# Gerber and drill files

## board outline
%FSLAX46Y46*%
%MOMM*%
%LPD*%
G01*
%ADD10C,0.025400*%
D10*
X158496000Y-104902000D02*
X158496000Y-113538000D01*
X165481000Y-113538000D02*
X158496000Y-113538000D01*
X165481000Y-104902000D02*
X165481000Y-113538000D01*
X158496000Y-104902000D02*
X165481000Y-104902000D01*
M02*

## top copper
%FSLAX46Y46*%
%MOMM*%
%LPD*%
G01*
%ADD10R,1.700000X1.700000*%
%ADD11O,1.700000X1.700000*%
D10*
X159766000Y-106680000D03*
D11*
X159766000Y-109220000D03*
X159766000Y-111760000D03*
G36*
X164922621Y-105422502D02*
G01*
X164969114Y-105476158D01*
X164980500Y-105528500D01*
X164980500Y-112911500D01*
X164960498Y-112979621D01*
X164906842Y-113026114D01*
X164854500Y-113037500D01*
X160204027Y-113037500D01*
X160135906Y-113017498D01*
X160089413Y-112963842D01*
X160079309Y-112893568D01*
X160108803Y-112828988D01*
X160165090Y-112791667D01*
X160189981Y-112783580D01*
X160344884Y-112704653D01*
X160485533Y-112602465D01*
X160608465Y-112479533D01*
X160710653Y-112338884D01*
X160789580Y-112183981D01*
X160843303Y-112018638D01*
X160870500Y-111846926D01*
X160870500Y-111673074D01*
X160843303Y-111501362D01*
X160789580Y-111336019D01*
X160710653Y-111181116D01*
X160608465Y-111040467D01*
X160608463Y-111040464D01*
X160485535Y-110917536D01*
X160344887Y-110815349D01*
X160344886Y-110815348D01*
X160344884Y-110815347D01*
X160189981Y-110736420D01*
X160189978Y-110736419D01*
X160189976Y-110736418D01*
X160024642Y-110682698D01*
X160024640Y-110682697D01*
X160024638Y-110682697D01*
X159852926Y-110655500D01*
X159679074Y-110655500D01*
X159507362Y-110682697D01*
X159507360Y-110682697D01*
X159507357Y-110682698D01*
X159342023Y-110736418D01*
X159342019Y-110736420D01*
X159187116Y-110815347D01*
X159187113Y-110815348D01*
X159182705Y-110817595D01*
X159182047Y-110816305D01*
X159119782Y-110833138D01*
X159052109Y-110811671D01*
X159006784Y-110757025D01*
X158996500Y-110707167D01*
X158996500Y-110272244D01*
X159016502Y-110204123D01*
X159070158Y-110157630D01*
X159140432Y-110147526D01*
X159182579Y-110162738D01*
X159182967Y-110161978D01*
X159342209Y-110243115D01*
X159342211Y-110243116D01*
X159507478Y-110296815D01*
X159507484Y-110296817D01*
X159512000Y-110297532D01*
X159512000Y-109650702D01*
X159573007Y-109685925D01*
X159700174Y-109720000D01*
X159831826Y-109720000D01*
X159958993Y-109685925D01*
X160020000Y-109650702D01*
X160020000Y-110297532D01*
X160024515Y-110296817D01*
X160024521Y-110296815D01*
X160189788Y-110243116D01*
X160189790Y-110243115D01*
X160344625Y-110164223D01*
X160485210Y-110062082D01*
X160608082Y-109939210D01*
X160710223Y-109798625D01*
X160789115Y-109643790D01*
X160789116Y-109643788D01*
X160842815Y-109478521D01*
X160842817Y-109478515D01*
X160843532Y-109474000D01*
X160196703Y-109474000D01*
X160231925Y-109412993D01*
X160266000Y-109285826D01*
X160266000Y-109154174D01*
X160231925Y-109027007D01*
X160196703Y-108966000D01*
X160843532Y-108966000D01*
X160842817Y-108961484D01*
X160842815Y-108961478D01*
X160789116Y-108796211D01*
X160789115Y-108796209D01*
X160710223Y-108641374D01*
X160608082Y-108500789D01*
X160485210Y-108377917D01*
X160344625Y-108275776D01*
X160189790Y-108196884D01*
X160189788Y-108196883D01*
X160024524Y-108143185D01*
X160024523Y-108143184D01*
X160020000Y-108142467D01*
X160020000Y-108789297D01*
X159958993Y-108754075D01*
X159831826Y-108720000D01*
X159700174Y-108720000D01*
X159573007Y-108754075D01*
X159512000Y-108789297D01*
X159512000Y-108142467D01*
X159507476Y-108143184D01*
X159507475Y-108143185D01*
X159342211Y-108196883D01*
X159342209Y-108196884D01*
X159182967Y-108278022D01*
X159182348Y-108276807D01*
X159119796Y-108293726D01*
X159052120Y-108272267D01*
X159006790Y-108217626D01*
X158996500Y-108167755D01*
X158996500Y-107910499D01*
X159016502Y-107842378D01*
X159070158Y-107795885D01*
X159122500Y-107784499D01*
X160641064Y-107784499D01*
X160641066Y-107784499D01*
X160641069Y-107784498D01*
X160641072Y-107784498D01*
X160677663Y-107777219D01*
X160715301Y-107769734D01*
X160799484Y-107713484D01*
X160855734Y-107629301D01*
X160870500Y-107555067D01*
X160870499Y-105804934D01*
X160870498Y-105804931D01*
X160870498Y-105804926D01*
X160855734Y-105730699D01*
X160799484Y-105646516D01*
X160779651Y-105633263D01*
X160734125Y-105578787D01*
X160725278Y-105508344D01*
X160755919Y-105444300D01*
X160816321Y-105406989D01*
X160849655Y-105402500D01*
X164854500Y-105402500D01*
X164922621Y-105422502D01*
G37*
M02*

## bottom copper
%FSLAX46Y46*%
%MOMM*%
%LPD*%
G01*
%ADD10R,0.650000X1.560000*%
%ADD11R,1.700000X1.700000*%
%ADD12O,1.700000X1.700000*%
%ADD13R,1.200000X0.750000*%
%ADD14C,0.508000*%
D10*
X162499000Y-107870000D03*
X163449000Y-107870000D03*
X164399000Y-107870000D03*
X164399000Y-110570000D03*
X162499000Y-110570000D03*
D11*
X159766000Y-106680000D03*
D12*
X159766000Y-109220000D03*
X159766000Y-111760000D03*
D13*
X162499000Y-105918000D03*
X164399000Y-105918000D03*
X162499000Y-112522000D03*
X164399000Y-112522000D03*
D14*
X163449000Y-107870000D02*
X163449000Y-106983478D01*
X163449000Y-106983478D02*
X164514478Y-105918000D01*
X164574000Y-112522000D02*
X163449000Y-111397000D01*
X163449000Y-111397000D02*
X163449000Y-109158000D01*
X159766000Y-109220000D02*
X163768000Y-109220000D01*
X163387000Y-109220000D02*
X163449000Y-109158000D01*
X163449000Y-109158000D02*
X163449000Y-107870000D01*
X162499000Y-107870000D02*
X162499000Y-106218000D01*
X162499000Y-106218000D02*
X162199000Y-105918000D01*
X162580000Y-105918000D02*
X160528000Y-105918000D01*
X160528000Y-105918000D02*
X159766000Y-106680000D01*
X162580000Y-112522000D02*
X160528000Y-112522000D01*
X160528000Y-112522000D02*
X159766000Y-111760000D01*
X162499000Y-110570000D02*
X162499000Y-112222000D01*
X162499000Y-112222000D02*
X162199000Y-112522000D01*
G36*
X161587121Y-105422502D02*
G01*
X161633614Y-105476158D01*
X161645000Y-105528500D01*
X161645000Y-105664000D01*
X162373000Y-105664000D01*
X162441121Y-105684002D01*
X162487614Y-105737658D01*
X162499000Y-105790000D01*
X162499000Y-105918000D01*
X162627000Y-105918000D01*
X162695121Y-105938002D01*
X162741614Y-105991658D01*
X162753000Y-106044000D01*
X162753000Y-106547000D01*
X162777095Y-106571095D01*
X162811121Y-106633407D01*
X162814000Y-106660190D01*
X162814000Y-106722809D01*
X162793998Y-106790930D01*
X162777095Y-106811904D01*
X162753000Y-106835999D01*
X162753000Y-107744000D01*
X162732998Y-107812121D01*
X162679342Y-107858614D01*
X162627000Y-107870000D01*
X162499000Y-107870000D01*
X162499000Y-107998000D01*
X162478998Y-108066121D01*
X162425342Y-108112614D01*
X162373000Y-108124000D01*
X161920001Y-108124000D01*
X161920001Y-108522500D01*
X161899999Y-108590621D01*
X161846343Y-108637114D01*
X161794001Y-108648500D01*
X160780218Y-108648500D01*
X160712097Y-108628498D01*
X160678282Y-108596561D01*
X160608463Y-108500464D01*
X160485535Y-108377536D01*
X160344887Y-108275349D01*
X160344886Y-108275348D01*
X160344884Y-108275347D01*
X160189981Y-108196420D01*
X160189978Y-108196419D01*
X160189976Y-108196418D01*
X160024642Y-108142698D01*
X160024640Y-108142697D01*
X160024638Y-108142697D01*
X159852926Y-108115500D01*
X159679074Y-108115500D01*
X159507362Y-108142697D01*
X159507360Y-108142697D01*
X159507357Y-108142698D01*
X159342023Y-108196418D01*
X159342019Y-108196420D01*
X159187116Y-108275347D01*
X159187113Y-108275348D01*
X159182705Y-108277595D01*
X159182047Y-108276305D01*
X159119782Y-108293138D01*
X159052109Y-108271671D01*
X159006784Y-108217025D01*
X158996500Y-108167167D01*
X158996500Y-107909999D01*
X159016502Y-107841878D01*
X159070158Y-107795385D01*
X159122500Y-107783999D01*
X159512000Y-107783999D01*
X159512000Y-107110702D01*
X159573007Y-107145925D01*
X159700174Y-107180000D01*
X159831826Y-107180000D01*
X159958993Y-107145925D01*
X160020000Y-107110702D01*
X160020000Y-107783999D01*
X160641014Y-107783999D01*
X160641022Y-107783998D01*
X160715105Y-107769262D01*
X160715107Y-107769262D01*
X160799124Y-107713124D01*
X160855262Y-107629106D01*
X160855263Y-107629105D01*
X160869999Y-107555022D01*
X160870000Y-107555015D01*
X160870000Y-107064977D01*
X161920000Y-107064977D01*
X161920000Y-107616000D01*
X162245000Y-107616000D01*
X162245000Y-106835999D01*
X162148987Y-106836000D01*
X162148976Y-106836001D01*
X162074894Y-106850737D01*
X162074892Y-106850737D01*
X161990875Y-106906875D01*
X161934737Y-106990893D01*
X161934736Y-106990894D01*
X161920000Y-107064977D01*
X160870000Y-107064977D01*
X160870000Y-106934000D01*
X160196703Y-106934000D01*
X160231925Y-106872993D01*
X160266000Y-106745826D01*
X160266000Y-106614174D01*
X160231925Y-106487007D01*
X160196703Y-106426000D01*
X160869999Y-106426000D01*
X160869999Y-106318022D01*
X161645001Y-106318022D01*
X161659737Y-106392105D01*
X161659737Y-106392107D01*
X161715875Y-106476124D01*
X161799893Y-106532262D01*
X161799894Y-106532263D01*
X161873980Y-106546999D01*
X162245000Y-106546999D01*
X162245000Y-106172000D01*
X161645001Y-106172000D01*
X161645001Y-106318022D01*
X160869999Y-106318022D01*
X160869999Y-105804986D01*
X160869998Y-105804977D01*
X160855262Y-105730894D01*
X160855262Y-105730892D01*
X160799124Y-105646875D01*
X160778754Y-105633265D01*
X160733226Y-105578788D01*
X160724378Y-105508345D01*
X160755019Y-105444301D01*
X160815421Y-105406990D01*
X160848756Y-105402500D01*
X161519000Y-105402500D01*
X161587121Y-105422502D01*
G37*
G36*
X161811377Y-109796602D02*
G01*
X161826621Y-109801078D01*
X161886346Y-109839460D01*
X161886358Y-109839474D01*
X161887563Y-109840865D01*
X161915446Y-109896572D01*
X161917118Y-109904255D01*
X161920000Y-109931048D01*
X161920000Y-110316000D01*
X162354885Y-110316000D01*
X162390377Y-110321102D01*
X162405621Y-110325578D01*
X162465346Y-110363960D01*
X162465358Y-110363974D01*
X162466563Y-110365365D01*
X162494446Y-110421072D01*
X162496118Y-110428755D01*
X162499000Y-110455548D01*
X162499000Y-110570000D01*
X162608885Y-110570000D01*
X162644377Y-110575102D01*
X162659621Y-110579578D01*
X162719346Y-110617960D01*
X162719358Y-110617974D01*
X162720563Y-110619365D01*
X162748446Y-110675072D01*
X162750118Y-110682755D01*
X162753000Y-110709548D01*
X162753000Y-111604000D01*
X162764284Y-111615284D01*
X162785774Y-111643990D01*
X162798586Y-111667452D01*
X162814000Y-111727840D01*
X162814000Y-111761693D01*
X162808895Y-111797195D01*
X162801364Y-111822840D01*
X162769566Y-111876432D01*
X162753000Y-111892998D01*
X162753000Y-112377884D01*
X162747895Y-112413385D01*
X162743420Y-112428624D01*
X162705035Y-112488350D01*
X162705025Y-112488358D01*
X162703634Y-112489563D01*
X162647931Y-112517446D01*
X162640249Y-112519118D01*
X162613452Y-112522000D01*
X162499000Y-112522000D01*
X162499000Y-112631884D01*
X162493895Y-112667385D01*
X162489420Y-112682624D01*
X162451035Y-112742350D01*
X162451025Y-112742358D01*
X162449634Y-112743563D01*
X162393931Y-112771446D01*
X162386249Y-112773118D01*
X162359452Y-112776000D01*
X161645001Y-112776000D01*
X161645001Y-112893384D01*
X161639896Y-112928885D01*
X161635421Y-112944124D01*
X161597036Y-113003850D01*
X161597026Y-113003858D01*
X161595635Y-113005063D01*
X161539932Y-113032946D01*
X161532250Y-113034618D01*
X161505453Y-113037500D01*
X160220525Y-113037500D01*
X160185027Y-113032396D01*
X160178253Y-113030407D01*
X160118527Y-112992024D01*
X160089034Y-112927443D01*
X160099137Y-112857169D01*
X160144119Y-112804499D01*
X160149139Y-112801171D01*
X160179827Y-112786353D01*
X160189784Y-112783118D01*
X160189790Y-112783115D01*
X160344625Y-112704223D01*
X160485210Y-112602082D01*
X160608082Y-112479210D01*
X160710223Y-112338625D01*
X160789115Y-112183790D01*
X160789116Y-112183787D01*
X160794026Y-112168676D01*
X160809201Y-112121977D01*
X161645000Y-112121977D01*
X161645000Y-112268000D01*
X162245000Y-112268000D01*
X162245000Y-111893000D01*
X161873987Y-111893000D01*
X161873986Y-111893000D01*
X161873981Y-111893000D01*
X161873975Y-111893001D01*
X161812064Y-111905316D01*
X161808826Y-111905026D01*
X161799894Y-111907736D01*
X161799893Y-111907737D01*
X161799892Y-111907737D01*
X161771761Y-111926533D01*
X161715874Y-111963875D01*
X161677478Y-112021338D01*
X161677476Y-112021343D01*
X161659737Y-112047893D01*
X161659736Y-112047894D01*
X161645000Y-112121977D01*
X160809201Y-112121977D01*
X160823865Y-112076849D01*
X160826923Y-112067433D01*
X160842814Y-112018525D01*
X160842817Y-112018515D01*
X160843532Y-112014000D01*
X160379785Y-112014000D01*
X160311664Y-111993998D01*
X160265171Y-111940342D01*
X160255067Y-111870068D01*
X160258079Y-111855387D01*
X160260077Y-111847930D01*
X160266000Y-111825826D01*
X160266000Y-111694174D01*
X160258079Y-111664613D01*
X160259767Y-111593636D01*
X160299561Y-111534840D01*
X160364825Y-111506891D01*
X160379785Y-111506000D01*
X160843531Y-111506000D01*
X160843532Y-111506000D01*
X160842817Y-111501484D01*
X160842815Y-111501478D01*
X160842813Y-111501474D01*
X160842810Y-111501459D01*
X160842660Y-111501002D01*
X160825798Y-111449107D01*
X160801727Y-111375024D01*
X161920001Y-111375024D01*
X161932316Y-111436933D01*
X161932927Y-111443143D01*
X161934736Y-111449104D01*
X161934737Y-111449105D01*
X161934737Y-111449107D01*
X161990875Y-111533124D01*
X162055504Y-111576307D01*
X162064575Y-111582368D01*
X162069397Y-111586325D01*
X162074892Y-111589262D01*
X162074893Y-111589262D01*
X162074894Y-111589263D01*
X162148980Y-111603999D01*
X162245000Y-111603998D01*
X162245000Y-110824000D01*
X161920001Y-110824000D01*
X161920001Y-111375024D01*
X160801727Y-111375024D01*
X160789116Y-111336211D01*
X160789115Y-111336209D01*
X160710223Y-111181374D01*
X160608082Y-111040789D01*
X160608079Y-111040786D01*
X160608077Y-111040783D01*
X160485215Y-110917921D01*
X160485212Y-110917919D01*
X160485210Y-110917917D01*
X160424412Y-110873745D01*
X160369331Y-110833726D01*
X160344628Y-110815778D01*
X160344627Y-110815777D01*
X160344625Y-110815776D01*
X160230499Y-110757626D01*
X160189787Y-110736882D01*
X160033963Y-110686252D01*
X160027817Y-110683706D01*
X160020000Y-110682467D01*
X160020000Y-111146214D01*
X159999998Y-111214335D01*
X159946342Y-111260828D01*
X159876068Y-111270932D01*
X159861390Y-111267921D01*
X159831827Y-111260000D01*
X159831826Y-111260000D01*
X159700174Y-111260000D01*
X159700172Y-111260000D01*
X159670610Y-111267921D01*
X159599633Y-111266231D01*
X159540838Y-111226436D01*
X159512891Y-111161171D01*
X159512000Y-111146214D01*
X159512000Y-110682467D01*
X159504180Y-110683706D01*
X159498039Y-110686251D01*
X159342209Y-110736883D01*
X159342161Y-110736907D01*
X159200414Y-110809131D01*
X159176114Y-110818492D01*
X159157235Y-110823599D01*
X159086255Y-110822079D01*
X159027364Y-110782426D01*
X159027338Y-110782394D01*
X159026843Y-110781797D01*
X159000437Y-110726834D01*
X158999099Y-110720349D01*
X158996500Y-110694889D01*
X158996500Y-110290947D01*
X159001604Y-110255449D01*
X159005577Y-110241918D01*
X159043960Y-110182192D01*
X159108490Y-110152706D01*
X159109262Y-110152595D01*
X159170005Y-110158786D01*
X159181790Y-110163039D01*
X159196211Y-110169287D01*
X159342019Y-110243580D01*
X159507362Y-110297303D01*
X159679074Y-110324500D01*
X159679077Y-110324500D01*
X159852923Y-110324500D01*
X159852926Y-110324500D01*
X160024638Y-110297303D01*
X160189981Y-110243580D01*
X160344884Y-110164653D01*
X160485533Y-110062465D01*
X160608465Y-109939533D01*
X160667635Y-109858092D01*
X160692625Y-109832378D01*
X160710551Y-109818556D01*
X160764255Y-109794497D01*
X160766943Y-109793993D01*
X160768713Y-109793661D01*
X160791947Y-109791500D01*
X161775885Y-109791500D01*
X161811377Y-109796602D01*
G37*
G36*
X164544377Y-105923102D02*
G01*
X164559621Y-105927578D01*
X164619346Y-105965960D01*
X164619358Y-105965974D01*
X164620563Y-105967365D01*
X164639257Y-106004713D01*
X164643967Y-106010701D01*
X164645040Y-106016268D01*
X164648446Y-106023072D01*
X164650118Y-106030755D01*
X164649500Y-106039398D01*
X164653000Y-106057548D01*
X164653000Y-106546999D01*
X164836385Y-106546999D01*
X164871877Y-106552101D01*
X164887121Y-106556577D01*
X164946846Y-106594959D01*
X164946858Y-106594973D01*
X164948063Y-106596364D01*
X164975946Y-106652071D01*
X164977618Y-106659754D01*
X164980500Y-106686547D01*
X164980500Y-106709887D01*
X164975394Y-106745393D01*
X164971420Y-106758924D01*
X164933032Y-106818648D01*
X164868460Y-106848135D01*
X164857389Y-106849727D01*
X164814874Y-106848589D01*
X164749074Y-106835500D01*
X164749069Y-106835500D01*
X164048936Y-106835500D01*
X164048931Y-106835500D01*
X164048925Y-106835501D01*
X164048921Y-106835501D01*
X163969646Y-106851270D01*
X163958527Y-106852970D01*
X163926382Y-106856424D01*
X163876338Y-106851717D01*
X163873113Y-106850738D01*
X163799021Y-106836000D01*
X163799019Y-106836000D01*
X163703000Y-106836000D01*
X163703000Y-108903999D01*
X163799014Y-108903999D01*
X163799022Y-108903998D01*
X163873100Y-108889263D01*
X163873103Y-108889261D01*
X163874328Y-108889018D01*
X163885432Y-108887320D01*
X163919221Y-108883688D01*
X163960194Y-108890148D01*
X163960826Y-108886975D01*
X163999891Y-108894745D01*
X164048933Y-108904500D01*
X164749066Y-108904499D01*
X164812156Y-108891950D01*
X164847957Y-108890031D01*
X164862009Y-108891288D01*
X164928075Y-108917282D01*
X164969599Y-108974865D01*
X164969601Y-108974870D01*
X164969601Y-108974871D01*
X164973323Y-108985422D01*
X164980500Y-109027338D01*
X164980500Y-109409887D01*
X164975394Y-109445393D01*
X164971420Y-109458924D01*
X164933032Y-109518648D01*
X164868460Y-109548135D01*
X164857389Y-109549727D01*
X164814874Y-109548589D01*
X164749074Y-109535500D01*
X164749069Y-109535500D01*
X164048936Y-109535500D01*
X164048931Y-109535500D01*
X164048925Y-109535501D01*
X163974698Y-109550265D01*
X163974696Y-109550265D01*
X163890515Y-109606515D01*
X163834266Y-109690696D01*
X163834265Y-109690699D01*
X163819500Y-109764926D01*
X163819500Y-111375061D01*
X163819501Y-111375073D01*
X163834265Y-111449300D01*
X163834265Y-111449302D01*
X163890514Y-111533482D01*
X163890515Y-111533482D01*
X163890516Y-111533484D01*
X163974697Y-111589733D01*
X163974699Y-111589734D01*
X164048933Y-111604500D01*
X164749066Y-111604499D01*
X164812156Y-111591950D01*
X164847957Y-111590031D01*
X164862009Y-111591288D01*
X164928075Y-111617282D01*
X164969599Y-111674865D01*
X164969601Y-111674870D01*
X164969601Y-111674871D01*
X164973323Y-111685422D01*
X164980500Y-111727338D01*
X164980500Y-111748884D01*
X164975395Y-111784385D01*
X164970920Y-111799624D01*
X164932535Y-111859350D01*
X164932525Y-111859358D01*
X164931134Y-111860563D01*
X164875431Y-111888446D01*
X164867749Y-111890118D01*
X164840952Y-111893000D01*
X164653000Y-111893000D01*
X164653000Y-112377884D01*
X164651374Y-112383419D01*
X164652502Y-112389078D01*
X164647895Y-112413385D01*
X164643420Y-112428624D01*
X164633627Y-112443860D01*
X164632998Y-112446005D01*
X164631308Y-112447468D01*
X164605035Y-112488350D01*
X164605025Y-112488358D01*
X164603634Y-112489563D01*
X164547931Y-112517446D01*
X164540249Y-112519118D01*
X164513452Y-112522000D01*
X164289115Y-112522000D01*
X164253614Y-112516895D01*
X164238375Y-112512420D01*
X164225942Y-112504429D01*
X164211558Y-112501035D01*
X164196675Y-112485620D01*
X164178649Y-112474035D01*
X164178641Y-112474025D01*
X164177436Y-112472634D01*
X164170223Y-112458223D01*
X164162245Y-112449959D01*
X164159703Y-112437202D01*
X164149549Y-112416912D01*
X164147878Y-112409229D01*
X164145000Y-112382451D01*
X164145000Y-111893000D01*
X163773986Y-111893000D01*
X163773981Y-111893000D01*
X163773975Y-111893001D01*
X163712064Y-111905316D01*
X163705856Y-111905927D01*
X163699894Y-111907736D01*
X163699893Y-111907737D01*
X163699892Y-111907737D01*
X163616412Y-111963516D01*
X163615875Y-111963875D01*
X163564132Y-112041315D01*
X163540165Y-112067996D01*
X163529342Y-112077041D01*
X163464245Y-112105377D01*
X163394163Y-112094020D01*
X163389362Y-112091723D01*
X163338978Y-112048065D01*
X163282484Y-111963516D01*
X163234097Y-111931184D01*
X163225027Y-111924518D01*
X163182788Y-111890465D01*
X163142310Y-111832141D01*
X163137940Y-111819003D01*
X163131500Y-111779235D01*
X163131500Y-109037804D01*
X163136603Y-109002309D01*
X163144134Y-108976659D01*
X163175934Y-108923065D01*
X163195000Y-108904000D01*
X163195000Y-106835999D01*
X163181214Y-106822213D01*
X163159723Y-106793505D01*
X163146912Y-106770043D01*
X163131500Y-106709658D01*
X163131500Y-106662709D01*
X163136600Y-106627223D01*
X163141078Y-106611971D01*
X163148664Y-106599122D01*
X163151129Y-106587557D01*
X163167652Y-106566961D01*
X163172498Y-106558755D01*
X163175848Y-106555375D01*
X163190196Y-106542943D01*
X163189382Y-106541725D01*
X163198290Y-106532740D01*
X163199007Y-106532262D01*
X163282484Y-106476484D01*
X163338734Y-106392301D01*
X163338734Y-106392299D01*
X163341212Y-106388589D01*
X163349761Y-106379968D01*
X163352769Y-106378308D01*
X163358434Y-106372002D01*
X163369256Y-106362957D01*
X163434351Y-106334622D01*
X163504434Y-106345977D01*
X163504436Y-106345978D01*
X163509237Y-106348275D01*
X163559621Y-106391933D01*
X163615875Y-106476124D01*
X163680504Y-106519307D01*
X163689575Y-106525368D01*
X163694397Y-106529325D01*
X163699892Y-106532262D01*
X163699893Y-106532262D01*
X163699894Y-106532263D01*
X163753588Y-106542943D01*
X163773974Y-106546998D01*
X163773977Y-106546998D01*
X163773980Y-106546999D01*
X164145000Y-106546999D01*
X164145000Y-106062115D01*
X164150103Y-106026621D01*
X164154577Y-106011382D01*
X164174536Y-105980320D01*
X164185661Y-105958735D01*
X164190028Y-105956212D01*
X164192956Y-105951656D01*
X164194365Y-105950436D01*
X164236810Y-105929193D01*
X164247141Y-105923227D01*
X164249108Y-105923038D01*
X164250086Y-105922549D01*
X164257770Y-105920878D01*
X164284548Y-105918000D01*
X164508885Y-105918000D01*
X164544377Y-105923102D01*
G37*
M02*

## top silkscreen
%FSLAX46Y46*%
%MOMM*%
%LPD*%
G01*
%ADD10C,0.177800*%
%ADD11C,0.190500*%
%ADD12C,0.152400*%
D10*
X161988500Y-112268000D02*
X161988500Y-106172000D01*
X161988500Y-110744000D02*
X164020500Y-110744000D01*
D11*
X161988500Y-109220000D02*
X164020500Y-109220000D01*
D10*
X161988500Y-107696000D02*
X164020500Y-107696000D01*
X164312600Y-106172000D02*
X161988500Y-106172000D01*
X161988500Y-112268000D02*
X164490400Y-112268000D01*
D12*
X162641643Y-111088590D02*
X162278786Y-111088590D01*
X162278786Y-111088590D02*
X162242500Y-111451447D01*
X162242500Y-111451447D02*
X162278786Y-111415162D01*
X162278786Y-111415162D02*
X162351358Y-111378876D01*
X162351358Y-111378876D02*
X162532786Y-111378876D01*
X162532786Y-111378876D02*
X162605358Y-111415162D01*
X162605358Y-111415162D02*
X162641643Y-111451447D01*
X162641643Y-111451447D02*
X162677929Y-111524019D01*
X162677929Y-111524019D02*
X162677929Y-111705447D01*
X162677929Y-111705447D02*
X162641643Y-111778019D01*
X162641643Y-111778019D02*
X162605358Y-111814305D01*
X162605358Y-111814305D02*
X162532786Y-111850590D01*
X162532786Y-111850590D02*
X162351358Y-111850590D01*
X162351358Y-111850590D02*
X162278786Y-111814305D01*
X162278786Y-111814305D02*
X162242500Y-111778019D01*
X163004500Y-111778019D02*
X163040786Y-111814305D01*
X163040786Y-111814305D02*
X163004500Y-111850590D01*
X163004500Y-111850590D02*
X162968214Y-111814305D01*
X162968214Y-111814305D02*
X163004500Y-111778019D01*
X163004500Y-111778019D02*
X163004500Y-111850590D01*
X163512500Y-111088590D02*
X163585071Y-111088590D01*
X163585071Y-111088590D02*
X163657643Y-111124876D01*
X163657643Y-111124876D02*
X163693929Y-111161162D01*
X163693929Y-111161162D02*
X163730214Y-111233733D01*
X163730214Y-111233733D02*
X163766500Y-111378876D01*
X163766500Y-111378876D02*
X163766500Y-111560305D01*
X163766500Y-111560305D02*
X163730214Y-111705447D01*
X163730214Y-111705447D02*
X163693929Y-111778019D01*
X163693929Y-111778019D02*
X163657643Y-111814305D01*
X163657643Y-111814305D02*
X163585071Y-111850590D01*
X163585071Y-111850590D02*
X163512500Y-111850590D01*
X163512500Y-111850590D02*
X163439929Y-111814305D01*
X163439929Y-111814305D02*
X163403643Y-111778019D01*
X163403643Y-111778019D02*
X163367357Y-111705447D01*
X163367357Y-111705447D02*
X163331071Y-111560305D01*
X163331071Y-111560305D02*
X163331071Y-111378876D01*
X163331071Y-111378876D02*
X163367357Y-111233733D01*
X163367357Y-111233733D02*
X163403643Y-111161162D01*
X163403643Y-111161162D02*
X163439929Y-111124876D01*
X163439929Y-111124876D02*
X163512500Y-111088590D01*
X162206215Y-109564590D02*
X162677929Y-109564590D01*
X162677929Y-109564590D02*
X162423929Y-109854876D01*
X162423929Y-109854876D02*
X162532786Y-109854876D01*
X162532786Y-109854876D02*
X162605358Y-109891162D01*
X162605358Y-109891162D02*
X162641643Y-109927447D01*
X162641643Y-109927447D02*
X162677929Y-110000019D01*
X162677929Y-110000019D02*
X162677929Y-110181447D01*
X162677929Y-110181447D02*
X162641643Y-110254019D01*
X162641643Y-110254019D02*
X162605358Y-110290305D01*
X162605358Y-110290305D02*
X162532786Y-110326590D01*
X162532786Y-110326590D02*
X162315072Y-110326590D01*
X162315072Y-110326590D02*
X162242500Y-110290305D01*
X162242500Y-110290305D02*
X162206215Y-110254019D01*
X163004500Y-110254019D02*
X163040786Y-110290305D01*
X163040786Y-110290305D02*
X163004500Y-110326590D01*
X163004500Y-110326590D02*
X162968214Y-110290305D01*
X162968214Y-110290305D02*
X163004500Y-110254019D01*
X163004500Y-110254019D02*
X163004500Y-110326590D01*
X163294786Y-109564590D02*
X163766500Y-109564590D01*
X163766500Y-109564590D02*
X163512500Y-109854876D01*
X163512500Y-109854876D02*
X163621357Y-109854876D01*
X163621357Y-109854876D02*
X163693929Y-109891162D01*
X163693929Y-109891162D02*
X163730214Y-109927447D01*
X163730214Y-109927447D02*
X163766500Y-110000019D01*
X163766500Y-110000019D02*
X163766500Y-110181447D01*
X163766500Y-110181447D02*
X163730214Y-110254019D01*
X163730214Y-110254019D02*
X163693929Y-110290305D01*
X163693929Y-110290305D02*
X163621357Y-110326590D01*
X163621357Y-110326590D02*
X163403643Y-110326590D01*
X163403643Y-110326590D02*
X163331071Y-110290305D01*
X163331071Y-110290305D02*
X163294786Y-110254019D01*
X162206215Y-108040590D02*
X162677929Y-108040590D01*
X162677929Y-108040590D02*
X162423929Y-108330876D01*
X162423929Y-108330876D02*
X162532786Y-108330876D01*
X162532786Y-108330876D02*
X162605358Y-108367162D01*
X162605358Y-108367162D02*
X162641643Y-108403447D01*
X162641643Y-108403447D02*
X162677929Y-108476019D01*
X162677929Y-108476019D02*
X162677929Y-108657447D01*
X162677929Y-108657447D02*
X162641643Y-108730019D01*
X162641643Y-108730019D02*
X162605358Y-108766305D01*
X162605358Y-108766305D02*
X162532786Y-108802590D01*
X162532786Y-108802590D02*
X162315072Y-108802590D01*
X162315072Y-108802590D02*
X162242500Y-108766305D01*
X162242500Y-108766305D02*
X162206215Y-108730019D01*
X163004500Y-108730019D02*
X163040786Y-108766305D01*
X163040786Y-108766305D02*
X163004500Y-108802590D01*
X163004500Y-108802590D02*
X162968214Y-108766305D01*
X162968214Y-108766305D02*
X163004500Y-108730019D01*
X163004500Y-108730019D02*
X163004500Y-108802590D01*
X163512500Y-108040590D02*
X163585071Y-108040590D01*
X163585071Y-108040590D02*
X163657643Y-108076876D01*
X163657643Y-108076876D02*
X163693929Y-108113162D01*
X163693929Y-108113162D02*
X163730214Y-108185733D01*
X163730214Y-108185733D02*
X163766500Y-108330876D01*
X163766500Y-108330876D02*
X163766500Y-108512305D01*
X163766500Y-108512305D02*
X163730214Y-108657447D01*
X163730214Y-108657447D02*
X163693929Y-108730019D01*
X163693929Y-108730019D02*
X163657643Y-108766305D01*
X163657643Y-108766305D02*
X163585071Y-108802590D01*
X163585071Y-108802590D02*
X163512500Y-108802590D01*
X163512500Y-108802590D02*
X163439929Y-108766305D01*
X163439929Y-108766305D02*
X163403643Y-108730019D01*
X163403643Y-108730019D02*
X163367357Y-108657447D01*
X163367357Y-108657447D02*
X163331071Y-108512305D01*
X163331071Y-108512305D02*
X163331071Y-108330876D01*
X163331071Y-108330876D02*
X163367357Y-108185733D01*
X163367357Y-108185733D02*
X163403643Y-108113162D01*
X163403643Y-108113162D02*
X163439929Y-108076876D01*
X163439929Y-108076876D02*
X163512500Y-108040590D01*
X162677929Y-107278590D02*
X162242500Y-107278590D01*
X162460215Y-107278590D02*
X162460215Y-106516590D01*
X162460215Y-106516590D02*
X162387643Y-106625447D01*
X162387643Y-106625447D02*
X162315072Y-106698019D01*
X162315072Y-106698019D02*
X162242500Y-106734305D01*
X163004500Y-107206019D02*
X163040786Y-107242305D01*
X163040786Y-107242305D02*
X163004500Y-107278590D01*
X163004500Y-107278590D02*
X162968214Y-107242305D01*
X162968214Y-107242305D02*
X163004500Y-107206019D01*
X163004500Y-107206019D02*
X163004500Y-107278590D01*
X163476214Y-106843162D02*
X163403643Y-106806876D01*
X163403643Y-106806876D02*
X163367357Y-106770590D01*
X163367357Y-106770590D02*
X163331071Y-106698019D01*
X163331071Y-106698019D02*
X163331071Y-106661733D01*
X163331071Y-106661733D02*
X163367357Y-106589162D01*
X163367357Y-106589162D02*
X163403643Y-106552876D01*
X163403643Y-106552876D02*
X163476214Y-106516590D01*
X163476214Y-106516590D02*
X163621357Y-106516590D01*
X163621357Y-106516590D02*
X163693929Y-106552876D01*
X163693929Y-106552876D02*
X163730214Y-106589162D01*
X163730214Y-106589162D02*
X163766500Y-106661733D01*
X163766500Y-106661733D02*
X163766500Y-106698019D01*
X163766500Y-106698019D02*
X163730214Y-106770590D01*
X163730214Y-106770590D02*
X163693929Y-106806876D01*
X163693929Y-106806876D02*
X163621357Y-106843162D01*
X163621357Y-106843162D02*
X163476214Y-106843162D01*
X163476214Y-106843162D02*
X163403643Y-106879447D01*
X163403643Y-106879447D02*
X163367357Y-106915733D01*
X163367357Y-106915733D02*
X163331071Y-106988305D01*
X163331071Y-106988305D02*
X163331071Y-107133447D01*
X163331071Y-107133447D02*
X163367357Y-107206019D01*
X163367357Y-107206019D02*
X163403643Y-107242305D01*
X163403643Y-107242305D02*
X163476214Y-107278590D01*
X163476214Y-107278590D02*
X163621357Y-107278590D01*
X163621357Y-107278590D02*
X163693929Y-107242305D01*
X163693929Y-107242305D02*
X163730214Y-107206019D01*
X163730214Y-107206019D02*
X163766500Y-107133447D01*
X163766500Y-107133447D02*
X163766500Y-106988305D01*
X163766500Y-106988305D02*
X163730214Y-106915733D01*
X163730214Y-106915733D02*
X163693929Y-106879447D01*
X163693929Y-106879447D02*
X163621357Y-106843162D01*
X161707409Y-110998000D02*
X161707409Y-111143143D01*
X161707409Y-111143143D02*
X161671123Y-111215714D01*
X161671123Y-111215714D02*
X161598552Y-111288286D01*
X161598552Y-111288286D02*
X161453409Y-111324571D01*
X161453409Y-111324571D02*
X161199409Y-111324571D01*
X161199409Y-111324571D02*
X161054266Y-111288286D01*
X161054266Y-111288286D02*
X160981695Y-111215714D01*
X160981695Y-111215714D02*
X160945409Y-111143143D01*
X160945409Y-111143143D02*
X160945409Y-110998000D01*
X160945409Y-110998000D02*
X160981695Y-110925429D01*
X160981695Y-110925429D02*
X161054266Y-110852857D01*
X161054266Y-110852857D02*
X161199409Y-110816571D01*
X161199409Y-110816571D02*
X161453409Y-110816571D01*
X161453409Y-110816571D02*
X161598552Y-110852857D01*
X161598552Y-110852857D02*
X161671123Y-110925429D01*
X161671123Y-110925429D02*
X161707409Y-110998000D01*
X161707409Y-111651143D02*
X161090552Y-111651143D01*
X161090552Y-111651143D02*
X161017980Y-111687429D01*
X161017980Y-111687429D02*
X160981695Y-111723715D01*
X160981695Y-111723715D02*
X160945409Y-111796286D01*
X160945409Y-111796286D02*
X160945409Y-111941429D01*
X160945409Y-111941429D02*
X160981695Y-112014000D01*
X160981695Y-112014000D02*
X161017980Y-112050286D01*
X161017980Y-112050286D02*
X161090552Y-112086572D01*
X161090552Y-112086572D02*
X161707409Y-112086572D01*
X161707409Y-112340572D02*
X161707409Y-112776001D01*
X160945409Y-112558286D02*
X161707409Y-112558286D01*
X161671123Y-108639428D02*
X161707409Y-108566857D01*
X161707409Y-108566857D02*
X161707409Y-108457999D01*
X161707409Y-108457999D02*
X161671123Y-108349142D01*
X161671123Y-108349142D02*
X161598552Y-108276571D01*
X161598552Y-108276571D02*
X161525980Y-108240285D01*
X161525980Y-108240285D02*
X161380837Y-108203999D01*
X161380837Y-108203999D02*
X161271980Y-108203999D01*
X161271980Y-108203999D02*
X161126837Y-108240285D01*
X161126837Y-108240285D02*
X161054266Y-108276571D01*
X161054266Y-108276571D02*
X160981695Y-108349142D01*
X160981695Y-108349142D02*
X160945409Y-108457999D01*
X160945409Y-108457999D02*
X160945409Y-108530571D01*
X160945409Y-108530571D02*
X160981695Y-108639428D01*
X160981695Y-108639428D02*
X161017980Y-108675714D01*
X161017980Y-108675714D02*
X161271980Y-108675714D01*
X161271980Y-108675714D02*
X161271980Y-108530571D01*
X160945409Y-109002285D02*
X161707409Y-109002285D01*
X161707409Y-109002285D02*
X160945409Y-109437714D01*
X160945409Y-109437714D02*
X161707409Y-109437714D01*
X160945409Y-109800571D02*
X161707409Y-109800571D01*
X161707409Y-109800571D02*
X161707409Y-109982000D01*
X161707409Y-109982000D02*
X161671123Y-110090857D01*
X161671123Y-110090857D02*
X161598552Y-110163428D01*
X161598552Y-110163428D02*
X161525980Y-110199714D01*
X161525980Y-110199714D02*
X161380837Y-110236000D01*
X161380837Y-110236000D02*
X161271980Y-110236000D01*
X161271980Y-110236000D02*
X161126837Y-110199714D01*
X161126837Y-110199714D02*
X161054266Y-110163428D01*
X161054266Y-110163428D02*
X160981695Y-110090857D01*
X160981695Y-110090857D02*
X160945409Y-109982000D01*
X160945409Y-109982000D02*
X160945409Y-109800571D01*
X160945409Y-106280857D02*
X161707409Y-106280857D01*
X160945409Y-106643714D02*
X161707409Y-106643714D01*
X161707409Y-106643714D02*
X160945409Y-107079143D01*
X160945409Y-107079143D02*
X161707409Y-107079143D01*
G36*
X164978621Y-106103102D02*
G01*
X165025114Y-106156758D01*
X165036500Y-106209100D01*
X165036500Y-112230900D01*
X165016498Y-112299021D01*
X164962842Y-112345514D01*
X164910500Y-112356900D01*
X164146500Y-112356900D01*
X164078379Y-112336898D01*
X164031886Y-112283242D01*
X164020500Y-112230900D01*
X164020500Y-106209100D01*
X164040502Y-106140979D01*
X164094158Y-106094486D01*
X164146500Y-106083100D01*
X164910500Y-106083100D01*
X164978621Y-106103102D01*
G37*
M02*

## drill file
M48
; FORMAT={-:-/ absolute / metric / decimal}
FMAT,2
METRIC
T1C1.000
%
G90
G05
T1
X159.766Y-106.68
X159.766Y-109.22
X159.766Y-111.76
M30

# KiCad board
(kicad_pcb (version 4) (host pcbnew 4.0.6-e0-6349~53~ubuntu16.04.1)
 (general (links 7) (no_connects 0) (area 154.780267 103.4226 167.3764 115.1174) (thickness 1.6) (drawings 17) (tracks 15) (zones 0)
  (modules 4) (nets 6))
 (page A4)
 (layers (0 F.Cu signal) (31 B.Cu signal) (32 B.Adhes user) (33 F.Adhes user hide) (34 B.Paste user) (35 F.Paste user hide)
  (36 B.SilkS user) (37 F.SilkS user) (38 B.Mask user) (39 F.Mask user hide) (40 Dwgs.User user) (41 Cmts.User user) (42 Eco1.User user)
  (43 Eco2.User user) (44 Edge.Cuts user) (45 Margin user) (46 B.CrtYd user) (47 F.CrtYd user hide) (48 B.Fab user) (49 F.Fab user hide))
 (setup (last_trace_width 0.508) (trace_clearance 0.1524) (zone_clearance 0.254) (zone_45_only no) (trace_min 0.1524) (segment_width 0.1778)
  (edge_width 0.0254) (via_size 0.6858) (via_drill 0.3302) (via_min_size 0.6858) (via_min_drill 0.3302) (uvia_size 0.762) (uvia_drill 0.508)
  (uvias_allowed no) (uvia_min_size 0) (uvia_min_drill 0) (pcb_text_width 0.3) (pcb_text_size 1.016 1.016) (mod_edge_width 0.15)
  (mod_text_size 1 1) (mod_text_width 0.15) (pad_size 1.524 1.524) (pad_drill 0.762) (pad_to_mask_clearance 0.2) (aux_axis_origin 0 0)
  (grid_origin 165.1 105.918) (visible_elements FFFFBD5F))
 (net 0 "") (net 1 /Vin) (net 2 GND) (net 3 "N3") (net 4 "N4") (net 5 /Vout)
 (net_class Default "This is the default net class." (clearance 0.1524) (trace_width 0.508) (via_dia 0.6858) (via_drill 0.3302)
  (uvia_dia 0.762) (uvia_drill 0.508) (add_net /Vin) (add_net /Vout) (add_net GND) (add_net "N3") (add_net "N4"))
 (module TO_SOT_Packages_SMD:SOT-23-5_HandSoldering (layer B.Cu) (at 163.449 109.22 270)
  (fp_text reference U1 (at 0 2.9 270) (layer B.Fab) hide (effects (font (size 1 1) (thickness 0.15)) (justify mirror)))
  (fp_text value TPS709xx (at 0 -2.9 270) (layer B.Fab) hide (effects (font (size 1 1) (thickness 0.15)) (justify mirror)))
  (pad 1 smd rect (at -1.35 0.95 270) (size 1.56 0.65) (layers B.Cu B.Paste B.Mask) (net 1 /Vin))
  (pad 2 smd rect (at -1.35 0 270) (size 1.56 0.65) (layers B.Cu B.Paste B.Mask) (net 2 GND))
  (pad 3 smd rect (at -1.35 -0.95 270) (size 1.56 0.65) (layers B.Cu B.Paste B.Mask) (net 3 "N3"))
  (pad 4 smd rect (at 1.35 -0.95 270) (size 1.56 0.65) (layers B.Cu B.Paste B.Mask) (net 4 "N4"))
  (pad 5 smd rect (at 1.35 0.95 270) (size 1.56 0.65) (layers B.Cu B.Paste B.Mask) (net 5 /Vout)))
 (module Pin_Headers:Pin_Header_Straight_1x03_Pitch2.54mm (layer B.Cu) (at 159.766 106.68 180)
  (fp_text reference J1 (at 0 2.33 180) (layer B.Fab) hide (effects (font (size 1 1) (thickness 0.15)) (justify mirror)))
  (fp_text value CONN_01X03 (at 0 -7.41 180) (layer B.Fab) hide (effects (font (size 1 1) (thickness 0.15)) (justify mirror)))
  (pad 1 thru_hole rect (at 0 0 180) (size 1.7 1.7) (drill 1) (layers *.Cu *.Mask) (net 1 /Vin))
  (pad 2 thru_hole oval (at 0 -2.54 180) (size 1.7 1.7) (drill 1) (layers *.Cu *.Mask) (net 2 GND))
  (pad 3 thru_hole oval (at 0 -5.08 180) (size 1.7 1.7) (drill 1) (layers *.Cu *.Mask) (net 5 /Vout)))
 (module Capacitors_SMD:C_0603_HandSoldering (layer B.Cu) (at 163.449 105.918)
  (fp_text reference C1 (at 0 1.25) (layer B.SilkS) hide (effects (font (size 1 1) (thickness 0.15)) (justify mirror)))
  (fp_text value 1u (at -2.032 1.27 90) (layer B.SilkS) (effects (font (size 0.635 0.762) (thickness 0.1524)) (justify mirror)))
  (pad 1 smd rect (at -0.95 0) (size 1.2 0.75) (layers B.Cu B.Paste B.Mask) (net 1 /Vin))
  (pad 2 smd rect (at 0.95 0) (size 1.2 0.75) (layers B.Cu B.Paste B.Mask) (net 2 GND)))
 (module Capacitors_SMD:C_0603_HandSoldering (layer B.Cu) (at 163.449 112.522)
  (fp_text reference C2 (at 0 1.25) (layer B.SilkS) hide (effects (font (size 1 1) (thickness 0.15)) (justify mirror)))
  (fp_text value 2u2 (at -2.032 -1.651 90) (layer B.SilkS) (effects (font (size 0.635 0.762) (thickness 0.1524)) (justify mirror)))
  (pad 1 smd rect (at -0.95 0) (size 1.2 0.75) (layers B.Cu B.Paste B.Mask) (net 5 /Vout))
  (pad 2 smd rect (at 0.95 0) (size 1.2 0.75) (layers B.Cu B.Paste B.Mask) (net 2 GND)))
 (gr_line (start 161.9885 112.268) (end 161.9885 106.172) (angle 90) (layer F.SilkS) (width 0.1778))
 (gr_line (start 161.9885 110.744) (end 164.0205 110.744) (angle 90) (layer F.SilkS) (width 0.1778))
 (gr_line (start 161.9885 109.22) (end 164.0205 109.22) (angle 90) (layer F.SilkS) (width 0.1905))
 (gr_line (start 161.9885 107.696) (end 164.0205 107.696) (angle 90) (layer F.SilkS) (width 0.1778))
 (gr_line (start 164.3126 106.172) (end 161.9885 106.172) (angle 90) (layer F.SilkS) (width 0.1778))
 (gr_line (start 161.9885 112.268) (end 164.4904 112.268) (angle 90) (layer F.SilkS) (width 0.1778))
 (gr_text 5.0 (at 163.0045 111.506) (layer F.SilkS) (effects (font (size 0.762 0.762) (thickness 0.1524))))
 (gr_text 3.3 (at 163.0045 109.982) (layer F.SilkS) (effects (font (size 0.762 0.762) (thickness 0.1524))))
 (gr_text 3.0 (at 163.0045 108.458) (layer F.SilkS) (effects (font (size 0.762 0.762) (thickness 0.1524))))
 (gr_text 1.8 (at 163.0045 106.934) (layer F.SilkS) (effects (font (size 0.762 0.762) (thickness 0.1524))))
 (gr_line (start 158.496 104.902) (end 158.496 113.538) (angle 90) (layer Edge.Cuts) (width 0.0254))
 (gr_line (start 165.481 113.538) (end 158.496 113.538) (angle 90) (layer Edge.Cuts) (width 0.0254))
 (gr_line (start 165.481 104.902) (end 165.481 113.538) (angle 90) (layer Edge.Cuts) (width 0.0254))
 (gr_line (start 158.496 104.902) (end 165.481 104.902) (angle 90) (layer Edge.Cuts) (width 0.0254))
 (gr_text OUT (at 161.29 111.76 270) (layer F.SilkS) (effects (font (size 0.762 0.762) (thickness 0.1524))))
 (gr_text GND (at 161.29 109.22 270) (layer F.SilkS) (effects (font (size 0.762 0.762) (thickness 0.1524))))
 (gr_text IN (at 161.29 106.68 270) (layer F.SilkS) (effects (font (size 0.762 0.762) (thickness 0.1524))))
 (segment (start 163.449 107.87) (end 163.449 106.983478) (width 0.508) (layer B.Cu) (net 2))
 (segment (start 163.449 106.983478) (end 164.514478 105.918) (width 0.508) (layer B.Cu) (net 2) (status 20))
 (segment (start 164.574 112.522) (end 163.449 111.397) (width 0.508) (layer B.Cu) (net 2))
 (segment (start 163.449 111.397) (end 163.449 109.158) (width 0.508) (layer B.Cu) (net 2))
 (segment (start 159.766 109.22) (end 163.768 109.22) (width 0.508) (layer B.Cu) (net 2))
 (segment (start 163.387 109.22) (end 163.449 109.158) (width 0.508) (layer B.Cu) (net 2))
 (segment (start 163.449 109.158) (end 163.449 107.87) (width 0.508) (layer B.Cu) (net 2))
 (segment (start 162.499 107.87) (end 162.499 106.218) (width 0.508) (layer B.Cu) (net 1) (status 20))
 (segment (start 162.499 106.218) (end 162.199 105.918) (width 0.508) (layer B.Cu) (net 1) (status 30))
 (segment (start 162.58 105.918) (end 160.528 105.918) (width 0.508) (layer B.Cu) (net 1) (status 10))
 (segment (start 160.528 105.918) (end 159.766 106.68) (width 0.508) (layer B.Cu) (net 1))
 (segment (start 162.58 112.522) (end 160.528 112.522) (width 0.508) (layer B.Cu) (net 5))
 (segment (start 160.528 112.522) (end 159.766 111.76) (width 0.508) (layer B.Cu) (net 5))
 (segment (start 162.499 110.57) (end 162.499 112.222) (width 0.508) (layer B.Cu) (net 5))
 (segment (start 162.499 112.222) (end 162.199 112.522) (width 0.508) (layer B.Cu) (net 5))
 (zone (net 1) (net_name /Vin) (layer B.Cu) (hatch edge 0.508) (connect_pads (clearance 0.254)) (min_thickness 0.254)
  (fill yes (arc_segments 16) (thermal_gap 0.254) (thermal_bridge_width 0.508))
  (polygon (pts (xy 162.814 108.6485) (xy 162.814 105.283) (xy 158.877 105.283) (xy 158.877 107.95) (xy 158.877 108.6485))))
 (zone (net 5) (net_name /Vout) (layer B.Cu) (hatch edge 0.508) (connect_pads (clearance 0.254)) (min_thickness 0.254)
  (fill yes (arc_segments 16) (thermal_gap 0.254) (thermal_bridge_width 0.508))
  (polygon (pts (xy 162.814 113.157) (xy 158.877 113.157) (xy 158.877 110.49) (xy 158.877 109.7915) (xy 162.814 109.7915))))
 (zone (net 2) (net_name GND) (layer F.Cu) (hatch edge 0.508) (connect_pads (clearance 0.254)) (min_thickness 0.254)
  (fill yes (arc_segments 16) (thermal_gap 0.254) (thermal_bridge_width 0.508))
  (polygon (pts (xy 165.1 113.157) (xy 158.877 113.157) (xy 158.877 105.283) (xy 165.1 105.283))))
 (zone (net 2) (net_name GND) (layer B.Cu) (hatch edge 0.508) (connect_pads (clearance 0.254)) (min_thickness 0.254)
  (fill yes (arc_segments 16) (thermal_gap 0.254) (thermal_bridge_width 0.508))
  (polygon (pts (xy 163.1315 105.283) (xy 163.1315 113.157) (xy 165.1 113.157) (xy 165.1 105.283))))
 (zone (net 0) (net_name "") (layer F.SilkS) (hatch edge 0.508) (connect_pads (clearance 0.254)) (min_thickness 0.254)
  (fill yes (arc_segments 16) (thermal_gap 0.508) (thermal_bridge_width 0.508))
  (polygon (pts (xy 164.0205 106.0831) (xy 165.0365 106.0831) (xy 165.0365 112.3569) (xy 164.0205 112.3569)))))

